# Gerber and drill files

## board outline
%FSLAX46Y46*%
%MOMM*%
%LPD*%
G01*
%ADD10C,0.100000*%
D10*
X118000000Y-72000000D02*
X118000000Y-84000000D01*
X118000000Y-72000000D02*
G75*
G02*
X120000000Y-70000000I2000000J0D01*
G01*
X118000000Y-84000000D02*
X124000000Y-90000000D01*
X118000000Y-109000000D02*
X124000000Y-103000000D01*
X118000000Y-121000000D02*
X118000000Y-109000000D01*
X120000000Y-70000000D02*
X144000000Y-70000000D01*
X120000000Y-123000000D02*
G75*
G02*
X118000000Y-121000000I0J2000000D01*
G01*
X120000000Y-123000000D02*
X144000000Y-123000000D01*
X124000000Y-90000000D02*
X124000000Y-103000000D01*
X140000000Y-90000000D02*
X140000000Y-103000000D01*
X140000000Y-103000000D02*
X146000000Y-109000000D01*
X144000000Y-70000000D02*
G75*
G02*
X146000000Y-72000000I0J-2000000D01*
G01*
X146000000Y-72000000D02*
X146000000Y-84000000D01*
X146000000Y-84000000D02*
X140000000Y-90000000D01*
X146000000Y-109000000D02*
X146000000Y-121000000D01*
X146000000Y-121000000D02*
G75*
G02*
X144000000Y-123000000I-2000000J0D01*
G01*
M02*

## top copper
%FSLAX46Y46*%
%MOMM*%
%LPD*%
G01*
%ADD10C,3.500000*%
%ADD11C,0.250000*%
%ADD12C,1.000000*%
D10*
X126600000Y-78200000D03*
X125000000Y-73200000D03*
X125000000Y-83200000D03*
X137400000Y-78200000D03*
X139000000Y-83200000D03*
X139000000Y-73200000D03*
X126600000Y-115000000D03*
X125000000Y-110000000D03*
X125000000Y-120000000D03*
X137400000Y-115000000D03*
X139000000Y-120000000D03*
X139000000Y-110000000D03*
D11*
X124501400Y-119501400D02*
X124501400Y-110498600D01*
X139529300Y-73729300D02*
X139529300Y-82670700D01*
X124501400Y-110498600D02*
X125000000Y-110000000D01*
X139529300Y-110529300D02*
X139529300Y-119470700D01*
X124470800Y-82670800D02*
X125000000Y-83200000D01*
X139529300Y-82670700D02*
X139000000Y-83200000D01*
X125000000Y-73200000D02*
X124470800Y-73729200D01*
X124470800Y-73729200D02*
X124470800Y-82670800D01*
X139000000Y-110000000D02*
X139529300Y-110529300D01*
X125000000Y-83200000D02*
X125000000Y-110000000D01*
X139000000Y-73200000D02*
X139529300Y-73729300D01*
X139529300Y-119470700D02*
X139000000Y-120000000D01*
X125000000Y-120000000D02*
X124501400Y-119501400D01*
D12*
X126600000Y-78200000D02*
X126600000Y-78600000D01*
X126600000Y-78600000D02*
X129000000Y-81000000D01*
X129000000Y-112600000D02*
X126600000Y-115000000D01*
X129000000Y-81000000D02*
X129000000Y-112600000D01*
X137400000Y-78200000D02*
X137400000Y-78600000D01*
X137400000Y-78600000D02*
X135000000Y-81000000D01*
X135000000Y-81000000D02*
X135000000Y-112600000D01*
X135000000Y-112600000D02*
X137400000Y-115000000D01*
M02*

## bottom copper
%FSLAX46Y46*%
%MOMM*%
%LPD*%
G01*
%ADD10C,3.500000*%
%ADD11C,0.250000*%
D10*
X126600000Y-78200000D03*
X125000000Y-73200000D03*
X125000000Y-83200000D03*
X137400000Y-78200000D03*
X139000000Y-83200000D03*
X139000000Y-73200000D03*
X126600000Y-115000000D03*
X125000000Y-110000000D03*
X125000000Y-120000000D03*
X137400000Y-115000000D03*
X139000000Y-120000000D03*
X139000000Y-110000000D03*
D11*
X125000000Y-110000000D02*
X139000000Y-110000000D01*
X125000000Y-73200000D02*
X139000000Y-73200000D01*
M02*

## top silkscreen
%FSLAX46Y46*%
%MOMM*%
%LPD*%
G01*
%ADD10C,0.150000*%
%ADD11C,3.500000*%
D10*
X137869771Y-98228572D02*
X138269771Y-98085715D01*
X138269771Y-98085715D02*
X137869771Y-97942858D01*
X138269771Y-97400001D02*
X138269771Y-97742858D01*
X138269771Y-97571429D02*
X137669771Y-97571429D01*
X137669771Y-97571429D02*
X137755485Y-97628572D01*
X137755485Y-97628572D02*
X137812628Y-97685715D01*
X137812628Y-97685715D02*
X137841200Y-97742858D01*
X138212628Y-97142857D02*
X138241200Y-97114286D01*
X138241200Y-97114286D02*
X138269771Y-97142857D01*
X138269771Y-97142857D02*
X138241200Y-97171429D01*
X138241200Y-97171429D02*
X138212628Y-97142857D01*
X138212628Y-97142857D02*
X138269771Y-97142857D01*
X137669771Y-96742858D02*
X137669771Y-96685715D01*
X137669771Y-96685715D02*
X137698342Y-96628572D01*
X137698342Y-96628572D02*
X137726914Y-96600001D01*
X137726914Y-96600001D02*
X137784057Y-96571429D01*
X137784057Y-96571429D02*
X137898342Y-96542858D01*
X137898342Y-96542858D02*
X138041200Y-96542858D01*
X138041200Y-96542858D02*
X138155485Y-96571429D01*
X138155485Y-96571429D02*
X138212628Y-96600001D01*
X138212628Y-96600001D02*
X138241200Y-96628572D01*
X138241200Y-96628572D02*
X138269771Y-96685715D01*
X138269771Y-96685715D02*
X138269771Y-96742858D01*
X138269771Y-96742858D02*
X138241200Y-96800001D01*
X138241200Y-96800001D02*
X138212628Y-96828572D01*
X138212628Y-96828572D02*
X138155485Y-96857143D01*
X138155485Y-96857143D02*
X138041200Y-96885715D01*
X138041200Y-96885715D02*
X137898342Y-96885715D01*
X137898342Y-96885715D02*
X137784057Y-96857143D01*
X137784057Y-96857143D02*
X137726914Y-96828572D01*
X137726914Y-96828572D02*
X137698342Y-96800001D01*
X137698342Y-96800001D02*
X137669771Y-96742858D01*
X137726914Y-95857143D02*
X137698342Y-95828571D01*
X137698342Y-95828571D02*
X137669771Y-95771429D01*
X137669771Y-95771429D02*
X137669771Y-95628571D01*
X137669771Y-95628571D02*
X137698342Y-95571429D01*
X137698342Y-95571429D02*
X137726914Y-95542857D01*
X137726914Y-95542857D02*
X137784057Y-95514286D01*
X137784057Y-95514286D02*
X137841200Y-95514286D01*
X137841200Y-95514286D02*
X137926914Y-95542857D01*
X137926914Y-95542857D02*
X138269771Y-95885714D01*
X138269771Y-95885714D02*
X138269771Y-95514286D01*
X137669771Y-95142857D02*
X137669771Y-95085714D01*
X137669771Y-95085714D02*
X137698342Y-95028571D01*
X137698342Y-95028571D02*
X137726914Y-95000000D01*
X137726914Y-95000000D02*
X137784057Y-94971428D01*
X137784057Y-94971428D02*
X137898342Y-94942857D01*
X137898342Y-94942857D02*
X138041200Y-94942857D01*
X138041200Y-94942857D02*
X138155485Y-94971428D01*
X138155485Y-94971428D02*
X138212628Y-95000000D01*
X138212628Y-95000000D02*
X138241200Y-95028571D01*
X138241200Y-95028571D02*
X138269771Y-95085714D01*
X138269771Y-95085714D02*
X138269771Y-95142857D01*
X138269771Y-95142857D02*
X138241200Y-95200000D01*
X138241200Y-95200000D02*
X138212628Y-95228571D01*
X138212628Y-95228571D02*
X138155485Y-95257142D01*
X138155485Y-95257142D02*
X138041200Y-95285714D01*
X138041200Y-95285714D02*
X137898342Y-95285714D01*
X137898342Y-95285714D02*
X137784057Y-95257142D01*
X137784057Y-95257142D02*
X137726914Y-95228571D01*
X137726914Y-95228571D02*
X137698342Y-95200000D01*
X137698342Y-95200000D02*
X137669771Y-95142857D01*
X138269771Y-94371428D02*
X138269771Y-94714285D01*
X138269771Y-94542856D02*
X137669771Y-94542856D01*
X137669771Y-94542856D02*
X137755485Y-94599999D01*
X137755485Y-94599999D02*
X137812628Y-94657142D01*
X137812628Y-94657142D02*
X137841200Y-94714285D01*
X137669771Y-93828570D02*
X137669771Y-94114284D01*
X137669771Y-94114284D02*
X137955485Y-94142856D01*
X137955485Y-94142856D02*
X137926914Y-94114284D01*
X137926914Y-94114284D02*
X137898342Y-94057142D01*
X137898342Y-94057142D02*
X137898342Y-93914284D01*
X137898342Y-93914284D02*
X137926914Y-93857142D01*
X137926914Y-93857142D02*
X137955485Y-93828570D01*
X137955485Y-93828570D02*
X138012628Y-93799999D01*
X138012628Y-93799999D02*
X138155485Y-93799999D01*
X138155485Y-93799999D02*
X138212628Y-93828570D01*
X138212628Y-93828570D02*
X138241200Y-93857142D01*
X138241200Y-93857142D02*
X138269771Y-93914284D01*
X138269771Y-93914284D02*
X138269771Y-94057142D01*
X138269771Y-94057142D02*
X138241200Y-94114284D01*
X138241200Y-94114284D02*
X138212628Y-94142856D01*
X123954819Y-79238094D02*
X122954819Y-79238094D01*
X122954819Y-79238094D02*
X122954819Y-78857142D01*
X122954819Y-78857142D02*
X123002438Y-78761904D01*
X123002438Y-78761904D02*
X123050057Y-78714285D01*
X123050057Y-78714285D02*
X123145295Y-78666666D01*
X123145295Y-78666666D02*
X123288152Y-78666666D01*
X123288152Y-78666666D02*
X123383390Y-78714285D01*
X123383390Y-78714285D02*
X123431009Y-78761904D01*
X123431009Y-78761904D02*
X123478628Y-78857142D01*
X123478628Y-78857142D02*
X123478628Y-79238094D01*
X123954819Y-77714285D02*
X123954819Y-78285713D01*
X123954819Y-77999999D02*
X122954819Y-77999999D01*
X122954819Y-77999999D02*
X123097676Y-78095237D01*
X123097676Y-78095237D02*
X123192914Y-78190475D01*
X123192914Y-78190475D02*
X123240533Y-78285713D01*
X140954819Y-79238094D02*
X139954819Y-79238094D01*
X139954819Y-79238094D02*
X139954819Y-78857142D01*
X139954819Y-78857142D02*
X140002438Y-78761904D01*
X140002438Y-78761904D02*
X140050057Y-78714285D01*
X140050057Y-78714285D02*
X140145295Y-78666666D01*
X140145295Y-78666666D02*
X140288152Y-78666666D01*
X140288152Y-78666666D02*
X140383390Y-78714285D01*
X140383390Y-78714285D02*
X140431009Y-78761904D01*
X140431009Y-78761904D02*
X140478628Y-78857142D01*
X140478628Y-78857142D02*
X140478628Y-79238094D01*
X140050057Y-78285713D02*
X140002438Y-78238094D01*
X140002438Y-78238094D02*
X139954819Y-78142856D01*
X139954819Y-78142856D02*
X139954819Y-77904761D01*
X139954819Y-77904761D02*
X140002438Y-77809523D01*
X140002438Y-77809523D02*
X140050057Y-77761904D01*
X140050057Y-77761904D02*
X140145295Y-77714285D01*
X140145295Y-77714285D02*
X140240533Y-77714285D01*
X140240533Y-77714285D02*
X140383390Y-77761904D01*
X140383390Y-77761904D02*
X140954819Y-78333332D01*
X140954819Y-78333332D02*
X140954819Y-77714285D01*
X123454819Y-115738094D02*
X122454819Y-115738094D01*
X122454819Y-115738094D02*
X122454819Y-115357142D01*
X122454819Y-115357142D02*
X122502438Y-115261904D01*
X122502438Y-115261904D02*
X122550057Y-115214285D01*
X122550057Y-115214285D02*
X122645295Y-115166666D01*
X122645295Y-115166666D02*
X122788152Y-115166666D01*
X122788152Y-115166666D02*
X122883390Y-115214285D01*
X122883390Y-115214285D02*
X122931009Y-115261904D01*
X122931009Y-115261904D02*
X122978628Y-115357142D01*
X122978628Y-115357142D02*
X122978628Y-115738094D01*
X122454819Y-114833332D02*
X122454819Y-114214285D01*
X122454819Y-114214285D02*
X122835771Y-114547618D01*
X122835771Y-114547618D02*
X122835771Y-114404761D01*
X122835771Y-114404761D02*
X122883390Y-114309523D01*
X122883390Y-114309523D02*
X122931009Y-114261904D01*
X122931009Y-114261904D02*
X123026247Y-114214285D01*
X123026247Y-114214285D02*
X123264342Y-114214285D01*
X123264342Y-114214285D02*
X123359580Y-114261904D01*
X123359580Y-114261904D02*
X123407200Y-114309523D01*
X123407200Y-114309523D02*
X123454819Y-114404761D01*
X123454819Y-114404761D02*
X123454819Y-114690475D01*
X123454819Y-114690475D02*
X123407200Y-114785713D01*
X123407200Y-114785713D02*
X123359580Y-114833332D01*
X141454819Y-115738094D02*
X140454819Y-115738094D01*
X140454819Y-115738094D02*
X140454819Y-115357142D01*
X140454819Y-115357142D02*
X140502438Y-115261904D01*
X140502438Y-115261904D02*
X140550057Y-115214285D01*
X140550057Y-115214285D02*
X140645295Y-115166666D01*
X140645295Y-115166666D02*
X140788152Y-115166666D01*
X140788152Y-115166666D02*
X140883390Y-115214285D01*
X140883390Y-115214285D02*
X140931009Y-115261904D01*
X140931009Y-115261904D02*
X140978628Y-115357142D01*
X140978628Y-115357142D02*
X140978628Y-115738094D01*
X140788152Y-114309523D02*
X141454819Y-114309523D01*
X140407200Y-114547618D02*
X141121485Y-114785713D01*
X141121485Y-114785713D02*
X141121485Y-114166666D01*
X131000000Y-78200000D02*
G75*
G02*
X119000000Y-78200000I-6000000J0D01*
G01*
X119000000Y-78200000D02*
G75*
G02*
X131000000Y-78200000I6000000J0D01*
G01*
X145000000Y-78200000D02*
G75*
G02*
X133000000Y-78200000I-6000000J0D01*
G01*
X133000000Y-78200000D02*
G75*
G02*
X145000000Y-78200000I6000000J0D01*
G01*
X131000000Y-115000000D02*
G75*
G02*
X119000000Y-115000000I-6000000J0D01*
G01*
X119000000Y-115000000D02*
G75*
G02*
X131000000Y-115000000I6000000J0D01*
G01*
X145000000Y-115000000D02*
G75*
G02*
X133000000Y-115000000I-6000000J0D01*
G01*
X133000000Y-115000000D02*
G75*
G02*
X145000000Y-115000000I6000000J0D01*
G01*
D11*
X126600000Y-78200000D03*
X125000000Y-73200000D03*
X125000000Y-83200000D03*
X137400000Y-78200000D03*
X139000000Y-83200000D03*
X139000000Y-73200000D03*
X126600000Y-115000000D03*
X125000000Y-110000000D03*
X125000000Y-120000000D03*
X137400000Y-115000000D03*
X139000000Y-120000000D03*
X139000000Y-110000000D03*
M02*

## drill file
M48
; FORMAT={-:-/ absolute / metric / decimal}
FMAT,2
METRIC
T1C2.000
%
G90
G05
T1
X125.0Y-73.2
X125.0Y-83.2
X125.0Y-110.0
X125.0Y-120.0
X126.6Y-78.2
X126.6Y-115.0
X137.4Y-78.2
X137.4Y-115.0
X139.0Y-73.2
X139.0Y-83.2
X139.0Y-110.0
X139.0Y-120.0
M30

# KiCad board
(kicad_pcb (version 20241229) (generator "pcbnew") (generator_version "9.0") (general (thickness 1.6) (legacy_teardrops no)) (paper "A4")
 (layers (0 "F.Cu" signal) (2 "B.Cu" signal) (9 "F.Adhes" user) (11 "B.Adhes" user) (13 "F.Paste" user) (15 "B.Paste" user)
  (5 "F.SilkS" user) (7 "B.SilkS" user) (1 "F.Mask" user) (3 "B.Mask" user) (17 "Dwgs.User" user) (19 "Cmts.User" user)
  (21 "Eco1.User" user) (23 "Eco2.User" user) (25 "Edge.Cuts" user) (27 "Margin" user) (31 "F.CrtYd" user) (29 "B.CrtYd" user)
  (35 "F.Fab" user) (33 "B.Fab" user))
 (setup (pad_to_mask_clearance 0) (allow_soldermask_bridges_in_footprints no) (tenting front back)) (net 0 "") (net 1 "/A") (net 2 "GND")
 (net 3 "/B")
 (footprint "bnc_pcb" (layer "F.Cu") (at 125 78.2 -90)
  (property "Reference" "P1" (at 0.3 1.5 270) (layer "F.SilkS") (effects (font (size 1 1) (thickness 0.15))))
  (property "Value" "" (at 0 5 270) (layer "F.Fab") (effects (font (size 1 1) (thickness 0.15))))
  (fp_circle (center 0 0) (end 6 0) (stroke (width 0.15) (type solid)) (fill no) (layer "F.SilkS"))
  (pad "1" thru_hole circle (at 0 -1.6 270) (size 3.5 3.5) (drill 2) (layers "*.Cu" "*.Mask" "F.SilkS") (remove_unused_layers no)
   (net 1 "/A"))
  (pad "2" thru_hole circle (at -5 0 270) (size 3.5 3.5) (drill 2) (layers "*.Cu" "*.Mask" "F.SilkS") (remove_unused_layers no)
   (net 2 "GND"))
  (pad "2" thru_hole circle (at 5 0 270) (size 3.5 3.5) (drill 2) (layers "*.Cu" "*.Mask" "F.SilkS") (remove_unused_layers no) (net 2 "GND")))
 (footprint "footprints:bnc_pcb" (layer "F.Cu") (at 139 78.2 90)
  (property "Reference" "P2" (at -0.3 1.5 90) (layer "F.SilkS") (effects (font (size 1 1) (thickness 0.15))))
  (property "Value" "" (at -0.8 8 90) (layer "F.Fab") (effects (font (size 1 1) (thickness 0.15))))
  (fp_circle (center 0 0) (end 6 0) (stroke (width 0.15) (type solid)) (fill no) (layer "F.SilkS"))
  (pad "1" thru_hole circle (at 0 -1.6 90) (size 3.5 3.5) (drill 2) (layers "*.Cu" "*.Mask" "F.SilkS") (remove_unused_layers no)
   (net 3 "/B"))
  (pad "2" thru_hole circle (at -5 0 90) (size 3.5 3.5) (drill 2) (layers "*.Cu" "*.Mask" "F.SilkS") (remove_unused_layers no) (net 2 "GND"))
  (pad "2" thru_hole circle (at 5 0 90) (size 3.5 3.5) (drill 2) (layers "*.Cu" "*.Mask" "F.SilkS") (remove_unused_layers no) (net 2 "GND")))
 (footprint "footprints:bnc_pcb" (layer "F.Cu") (at 125 115 -90)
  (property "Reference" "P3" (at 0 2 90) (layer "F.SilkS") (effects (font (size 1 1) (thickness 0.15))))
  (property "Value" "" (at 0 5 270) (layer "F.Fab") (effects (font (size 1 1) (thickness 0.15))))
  (fp_circle (center 0 0) (end 6 0) (stroke (width 0.15) (type solid)) (fill no) (layer "F.SilkS"))
  (pad "1" thru_hole circle (at 0 -1.6 270) (size 3.5 3.5) (drill 2) (layers "*.Cu" "*.Mask" "F.SilkS") (remove_unused_layers no)
   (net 1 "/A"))
  (pad "2" thru_hole circle (at -5 0 270) (size 3.5 3.5) (drill 2) (layers "*.Cu" "*.Mask" "F.SilkS") (remove_unused_layers no)
   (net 2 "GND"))
  (pad "2" thru_hole circle (at 5 0 270) (size 3.5 3.5) (drill 2) (layers "*.Cu" "*.Mask" "F.SilkS") (remove_unused_layers no) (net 2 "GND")))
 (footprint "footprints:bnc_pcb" (layer "F.Cu") (at 139 115 90)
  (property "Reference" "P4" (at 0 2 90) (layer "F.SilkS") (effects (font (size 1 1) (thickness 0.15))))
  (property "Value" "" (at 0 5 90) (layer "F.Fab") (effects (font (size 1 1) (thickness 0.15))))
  (fp_circle (center 0 0) (end 6 0) (stroke (width 0.15) (type solid)) (fill no) (layer "F.SilkS"))
  (pad "1" thru_hole circle (at 0 -1.6 90) (size 3.5 3.5) (drill 2) (layers "*.Cu" "*.Mask" "F.SilkS") (remove_unused_layers no)
   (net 3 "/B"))
  (pad "2" thru_hole circle (at -5 0 90) (size 3.5 3.5) (drill 2) (layers "*.Cu" "*.Mask" "F.SilkS") (remove_unused_layers no) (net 2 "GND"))
  (pad "2" thru_hole circle (at 5 0 90) (size 3.5 3.5) (drill 2) (layers "*.Cu" "*.Mask" "F.SilkS") (remove_unused_layers no) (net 2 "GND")))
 (gr_line (start 118 72) (end 118 84) (stroke (width 0.1) (type solid)) (layer "Edge.Cuts"))
 (gr_arc (start 118 72) (mid 118.585786 70.585786) (end 120 70) (stroke (width 0.1) (type solid)) (layer "Edge.Cuts"))
 (gr_line (start 118 84) (end 124 90) (stroke (width 0.1) (type solid)) (layer "Edge.Cuts"))
 (gr_line (start 118 109) (end 124 103) (stroke (width 0.1) (type solid)) (layer "Edge.Cuts"))
 (gr_line (start 118 121) (end 118 109) (stroke (width 0.1) (type solid)) (layer "Edge.Cuts"))
 (gr_line (start 120 70) (end 144 70) (stroke (width 0.1) (type solid)) (layer "Edge.Cuts"))
 (gr_arc (start 120 123) (mid 118.585786 122.414214) (end 118 121) (stroke (width 0.1) (type solid)) (layer "Edge.Cuts"))
 (gr_line (start 120 123) (end 144 123) (stroke (width 0.1) (type solid)) (layer "Edge.Cuts"))
 (gr_line (start 124 90) (end 124 103) (stroke (width 0.1) (type solid)) (layer "Edge.Cuts"))
 (gr_line (start 140 90) (end 140 103) (stroke (width 0.1) (type solid)) (layer "Edge.Cuts"))
 (gr_line (start 140 103) (end 146 109) (stroke (width 0.1) (type solid)) (layer "Edge.Cuts"))
 (gr_arc (start 144 70) (mid 145.414214 70.585786) (end 146 72) (stroke (width 0.1) (type solid)) (layer "Edge.Cuts"))
 (gr_line (start 146 72) (end 146 84) (stroke (width 0.1) (type solid)) (layer "Edge.Cuts"))
 (gr_line (start 146 84) (end 140 90) (stroke (width 0.1) (type solid)) (layer "Edge.Cuts"))
 (gr_line (start 146 109) (end 146 121) (stroke (width 0.1) (type solid)) (layer "Edge.Cuts"))
 (gr_arc (start 146 121) (mid 145.414214 122.414214) (end 144 123) (stroke (width 0.1) (type solid)) (layer "Edge.Cuts"))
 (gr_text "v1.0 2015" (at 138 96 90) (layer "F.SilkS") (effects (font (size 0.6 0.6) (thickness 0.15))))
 (segment (start 124.5014 119.5014) (end 124.5014 110.4986) (width 0.25) (layer "F.Cu") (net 2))
 (segment (start 139.5293 73.7293) (end 139.5293 82.6707) (width 0.25) (layer "F.Cu") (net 2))
 (segment (start 124.5014 110.4986) (end 125 110) (width 0.25) (layer "F.Cu") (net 2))
 (segment (start 139.5293 110.5293) (end 139.5293 119.4707) (width 0.25) (layer "F.Cu") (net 2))
 (segment (start 124.4708 82.6708) (end 125 83.2) (width 0.25) (layer "F.Cu") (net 2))
 (segment (start 139.5293 82.6707) (end 139 83.2) (width 0.25) (layer "F.Cu") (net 2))
 (segment (start 125 73.2) (end 124.4708 73.7292) (width 0.25) (layer "F.Cu") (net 2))
 (segment (start 124.4708 73.7292) (end 124.4708 82.6708) (width 0.25) (layer "F.Cu") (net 2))
 (segment (start 139 110) (end 139.5293 110.5293) (width 0.25) (layer "F.Cu") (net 2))
 (segment (start 125 83.2) (end 125 110) (width 0.25) (layer "F.Cu") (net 2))
 (segment (start 139 73.2) (end 139.5293 73.7293) (width 0.25) (layer "F.Cu") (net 2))
 (segment (start 139.5293 119.4707) (end 139 120) (width 0.25) (layer "F.Cu") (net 2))
 (segment (start 125 120) (end 124.5014 119.5014) (width 0.25) (layer "F.Cu") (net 2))
 (segment (start 125 110) (end 139 110) (width 0.25) (layer "B.Cu") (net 2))
 (segment (start 125 73.2) (end 139 73.2) (width 0.25) (layer "B.Cu") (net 2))
 (segment (start 126.6 78.2) (end 126.6 78.6) (width 1) (layer "F.Cu") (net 1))
 (segment (start 126.6 78.6) (end 129 81) (width 1) (layer "F.Cu") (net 1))
 (segment (start 129 112.6) (end 126.6 115) (width 1) (layer "F.Cu") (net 1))
 (segment (start 129 81) (end 129 112.6) (width 1) (layer "F.Cu") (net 1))
 (segment (start 137.4 78.2) (end 137.4 78.6) (width 1) (layer "F.Cu") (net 3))
 (segment (start 137.4 78.6) (end 135 81) (width 1) (layer "F.Cu") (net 3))
 (segment (start 135 81) (end 135 112.6) (width 1) (layer "F.Cu") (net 3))
 (segment (start 135 112.6) (end 137.4 115) (width 1) (layer "F.Cu") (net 3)))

